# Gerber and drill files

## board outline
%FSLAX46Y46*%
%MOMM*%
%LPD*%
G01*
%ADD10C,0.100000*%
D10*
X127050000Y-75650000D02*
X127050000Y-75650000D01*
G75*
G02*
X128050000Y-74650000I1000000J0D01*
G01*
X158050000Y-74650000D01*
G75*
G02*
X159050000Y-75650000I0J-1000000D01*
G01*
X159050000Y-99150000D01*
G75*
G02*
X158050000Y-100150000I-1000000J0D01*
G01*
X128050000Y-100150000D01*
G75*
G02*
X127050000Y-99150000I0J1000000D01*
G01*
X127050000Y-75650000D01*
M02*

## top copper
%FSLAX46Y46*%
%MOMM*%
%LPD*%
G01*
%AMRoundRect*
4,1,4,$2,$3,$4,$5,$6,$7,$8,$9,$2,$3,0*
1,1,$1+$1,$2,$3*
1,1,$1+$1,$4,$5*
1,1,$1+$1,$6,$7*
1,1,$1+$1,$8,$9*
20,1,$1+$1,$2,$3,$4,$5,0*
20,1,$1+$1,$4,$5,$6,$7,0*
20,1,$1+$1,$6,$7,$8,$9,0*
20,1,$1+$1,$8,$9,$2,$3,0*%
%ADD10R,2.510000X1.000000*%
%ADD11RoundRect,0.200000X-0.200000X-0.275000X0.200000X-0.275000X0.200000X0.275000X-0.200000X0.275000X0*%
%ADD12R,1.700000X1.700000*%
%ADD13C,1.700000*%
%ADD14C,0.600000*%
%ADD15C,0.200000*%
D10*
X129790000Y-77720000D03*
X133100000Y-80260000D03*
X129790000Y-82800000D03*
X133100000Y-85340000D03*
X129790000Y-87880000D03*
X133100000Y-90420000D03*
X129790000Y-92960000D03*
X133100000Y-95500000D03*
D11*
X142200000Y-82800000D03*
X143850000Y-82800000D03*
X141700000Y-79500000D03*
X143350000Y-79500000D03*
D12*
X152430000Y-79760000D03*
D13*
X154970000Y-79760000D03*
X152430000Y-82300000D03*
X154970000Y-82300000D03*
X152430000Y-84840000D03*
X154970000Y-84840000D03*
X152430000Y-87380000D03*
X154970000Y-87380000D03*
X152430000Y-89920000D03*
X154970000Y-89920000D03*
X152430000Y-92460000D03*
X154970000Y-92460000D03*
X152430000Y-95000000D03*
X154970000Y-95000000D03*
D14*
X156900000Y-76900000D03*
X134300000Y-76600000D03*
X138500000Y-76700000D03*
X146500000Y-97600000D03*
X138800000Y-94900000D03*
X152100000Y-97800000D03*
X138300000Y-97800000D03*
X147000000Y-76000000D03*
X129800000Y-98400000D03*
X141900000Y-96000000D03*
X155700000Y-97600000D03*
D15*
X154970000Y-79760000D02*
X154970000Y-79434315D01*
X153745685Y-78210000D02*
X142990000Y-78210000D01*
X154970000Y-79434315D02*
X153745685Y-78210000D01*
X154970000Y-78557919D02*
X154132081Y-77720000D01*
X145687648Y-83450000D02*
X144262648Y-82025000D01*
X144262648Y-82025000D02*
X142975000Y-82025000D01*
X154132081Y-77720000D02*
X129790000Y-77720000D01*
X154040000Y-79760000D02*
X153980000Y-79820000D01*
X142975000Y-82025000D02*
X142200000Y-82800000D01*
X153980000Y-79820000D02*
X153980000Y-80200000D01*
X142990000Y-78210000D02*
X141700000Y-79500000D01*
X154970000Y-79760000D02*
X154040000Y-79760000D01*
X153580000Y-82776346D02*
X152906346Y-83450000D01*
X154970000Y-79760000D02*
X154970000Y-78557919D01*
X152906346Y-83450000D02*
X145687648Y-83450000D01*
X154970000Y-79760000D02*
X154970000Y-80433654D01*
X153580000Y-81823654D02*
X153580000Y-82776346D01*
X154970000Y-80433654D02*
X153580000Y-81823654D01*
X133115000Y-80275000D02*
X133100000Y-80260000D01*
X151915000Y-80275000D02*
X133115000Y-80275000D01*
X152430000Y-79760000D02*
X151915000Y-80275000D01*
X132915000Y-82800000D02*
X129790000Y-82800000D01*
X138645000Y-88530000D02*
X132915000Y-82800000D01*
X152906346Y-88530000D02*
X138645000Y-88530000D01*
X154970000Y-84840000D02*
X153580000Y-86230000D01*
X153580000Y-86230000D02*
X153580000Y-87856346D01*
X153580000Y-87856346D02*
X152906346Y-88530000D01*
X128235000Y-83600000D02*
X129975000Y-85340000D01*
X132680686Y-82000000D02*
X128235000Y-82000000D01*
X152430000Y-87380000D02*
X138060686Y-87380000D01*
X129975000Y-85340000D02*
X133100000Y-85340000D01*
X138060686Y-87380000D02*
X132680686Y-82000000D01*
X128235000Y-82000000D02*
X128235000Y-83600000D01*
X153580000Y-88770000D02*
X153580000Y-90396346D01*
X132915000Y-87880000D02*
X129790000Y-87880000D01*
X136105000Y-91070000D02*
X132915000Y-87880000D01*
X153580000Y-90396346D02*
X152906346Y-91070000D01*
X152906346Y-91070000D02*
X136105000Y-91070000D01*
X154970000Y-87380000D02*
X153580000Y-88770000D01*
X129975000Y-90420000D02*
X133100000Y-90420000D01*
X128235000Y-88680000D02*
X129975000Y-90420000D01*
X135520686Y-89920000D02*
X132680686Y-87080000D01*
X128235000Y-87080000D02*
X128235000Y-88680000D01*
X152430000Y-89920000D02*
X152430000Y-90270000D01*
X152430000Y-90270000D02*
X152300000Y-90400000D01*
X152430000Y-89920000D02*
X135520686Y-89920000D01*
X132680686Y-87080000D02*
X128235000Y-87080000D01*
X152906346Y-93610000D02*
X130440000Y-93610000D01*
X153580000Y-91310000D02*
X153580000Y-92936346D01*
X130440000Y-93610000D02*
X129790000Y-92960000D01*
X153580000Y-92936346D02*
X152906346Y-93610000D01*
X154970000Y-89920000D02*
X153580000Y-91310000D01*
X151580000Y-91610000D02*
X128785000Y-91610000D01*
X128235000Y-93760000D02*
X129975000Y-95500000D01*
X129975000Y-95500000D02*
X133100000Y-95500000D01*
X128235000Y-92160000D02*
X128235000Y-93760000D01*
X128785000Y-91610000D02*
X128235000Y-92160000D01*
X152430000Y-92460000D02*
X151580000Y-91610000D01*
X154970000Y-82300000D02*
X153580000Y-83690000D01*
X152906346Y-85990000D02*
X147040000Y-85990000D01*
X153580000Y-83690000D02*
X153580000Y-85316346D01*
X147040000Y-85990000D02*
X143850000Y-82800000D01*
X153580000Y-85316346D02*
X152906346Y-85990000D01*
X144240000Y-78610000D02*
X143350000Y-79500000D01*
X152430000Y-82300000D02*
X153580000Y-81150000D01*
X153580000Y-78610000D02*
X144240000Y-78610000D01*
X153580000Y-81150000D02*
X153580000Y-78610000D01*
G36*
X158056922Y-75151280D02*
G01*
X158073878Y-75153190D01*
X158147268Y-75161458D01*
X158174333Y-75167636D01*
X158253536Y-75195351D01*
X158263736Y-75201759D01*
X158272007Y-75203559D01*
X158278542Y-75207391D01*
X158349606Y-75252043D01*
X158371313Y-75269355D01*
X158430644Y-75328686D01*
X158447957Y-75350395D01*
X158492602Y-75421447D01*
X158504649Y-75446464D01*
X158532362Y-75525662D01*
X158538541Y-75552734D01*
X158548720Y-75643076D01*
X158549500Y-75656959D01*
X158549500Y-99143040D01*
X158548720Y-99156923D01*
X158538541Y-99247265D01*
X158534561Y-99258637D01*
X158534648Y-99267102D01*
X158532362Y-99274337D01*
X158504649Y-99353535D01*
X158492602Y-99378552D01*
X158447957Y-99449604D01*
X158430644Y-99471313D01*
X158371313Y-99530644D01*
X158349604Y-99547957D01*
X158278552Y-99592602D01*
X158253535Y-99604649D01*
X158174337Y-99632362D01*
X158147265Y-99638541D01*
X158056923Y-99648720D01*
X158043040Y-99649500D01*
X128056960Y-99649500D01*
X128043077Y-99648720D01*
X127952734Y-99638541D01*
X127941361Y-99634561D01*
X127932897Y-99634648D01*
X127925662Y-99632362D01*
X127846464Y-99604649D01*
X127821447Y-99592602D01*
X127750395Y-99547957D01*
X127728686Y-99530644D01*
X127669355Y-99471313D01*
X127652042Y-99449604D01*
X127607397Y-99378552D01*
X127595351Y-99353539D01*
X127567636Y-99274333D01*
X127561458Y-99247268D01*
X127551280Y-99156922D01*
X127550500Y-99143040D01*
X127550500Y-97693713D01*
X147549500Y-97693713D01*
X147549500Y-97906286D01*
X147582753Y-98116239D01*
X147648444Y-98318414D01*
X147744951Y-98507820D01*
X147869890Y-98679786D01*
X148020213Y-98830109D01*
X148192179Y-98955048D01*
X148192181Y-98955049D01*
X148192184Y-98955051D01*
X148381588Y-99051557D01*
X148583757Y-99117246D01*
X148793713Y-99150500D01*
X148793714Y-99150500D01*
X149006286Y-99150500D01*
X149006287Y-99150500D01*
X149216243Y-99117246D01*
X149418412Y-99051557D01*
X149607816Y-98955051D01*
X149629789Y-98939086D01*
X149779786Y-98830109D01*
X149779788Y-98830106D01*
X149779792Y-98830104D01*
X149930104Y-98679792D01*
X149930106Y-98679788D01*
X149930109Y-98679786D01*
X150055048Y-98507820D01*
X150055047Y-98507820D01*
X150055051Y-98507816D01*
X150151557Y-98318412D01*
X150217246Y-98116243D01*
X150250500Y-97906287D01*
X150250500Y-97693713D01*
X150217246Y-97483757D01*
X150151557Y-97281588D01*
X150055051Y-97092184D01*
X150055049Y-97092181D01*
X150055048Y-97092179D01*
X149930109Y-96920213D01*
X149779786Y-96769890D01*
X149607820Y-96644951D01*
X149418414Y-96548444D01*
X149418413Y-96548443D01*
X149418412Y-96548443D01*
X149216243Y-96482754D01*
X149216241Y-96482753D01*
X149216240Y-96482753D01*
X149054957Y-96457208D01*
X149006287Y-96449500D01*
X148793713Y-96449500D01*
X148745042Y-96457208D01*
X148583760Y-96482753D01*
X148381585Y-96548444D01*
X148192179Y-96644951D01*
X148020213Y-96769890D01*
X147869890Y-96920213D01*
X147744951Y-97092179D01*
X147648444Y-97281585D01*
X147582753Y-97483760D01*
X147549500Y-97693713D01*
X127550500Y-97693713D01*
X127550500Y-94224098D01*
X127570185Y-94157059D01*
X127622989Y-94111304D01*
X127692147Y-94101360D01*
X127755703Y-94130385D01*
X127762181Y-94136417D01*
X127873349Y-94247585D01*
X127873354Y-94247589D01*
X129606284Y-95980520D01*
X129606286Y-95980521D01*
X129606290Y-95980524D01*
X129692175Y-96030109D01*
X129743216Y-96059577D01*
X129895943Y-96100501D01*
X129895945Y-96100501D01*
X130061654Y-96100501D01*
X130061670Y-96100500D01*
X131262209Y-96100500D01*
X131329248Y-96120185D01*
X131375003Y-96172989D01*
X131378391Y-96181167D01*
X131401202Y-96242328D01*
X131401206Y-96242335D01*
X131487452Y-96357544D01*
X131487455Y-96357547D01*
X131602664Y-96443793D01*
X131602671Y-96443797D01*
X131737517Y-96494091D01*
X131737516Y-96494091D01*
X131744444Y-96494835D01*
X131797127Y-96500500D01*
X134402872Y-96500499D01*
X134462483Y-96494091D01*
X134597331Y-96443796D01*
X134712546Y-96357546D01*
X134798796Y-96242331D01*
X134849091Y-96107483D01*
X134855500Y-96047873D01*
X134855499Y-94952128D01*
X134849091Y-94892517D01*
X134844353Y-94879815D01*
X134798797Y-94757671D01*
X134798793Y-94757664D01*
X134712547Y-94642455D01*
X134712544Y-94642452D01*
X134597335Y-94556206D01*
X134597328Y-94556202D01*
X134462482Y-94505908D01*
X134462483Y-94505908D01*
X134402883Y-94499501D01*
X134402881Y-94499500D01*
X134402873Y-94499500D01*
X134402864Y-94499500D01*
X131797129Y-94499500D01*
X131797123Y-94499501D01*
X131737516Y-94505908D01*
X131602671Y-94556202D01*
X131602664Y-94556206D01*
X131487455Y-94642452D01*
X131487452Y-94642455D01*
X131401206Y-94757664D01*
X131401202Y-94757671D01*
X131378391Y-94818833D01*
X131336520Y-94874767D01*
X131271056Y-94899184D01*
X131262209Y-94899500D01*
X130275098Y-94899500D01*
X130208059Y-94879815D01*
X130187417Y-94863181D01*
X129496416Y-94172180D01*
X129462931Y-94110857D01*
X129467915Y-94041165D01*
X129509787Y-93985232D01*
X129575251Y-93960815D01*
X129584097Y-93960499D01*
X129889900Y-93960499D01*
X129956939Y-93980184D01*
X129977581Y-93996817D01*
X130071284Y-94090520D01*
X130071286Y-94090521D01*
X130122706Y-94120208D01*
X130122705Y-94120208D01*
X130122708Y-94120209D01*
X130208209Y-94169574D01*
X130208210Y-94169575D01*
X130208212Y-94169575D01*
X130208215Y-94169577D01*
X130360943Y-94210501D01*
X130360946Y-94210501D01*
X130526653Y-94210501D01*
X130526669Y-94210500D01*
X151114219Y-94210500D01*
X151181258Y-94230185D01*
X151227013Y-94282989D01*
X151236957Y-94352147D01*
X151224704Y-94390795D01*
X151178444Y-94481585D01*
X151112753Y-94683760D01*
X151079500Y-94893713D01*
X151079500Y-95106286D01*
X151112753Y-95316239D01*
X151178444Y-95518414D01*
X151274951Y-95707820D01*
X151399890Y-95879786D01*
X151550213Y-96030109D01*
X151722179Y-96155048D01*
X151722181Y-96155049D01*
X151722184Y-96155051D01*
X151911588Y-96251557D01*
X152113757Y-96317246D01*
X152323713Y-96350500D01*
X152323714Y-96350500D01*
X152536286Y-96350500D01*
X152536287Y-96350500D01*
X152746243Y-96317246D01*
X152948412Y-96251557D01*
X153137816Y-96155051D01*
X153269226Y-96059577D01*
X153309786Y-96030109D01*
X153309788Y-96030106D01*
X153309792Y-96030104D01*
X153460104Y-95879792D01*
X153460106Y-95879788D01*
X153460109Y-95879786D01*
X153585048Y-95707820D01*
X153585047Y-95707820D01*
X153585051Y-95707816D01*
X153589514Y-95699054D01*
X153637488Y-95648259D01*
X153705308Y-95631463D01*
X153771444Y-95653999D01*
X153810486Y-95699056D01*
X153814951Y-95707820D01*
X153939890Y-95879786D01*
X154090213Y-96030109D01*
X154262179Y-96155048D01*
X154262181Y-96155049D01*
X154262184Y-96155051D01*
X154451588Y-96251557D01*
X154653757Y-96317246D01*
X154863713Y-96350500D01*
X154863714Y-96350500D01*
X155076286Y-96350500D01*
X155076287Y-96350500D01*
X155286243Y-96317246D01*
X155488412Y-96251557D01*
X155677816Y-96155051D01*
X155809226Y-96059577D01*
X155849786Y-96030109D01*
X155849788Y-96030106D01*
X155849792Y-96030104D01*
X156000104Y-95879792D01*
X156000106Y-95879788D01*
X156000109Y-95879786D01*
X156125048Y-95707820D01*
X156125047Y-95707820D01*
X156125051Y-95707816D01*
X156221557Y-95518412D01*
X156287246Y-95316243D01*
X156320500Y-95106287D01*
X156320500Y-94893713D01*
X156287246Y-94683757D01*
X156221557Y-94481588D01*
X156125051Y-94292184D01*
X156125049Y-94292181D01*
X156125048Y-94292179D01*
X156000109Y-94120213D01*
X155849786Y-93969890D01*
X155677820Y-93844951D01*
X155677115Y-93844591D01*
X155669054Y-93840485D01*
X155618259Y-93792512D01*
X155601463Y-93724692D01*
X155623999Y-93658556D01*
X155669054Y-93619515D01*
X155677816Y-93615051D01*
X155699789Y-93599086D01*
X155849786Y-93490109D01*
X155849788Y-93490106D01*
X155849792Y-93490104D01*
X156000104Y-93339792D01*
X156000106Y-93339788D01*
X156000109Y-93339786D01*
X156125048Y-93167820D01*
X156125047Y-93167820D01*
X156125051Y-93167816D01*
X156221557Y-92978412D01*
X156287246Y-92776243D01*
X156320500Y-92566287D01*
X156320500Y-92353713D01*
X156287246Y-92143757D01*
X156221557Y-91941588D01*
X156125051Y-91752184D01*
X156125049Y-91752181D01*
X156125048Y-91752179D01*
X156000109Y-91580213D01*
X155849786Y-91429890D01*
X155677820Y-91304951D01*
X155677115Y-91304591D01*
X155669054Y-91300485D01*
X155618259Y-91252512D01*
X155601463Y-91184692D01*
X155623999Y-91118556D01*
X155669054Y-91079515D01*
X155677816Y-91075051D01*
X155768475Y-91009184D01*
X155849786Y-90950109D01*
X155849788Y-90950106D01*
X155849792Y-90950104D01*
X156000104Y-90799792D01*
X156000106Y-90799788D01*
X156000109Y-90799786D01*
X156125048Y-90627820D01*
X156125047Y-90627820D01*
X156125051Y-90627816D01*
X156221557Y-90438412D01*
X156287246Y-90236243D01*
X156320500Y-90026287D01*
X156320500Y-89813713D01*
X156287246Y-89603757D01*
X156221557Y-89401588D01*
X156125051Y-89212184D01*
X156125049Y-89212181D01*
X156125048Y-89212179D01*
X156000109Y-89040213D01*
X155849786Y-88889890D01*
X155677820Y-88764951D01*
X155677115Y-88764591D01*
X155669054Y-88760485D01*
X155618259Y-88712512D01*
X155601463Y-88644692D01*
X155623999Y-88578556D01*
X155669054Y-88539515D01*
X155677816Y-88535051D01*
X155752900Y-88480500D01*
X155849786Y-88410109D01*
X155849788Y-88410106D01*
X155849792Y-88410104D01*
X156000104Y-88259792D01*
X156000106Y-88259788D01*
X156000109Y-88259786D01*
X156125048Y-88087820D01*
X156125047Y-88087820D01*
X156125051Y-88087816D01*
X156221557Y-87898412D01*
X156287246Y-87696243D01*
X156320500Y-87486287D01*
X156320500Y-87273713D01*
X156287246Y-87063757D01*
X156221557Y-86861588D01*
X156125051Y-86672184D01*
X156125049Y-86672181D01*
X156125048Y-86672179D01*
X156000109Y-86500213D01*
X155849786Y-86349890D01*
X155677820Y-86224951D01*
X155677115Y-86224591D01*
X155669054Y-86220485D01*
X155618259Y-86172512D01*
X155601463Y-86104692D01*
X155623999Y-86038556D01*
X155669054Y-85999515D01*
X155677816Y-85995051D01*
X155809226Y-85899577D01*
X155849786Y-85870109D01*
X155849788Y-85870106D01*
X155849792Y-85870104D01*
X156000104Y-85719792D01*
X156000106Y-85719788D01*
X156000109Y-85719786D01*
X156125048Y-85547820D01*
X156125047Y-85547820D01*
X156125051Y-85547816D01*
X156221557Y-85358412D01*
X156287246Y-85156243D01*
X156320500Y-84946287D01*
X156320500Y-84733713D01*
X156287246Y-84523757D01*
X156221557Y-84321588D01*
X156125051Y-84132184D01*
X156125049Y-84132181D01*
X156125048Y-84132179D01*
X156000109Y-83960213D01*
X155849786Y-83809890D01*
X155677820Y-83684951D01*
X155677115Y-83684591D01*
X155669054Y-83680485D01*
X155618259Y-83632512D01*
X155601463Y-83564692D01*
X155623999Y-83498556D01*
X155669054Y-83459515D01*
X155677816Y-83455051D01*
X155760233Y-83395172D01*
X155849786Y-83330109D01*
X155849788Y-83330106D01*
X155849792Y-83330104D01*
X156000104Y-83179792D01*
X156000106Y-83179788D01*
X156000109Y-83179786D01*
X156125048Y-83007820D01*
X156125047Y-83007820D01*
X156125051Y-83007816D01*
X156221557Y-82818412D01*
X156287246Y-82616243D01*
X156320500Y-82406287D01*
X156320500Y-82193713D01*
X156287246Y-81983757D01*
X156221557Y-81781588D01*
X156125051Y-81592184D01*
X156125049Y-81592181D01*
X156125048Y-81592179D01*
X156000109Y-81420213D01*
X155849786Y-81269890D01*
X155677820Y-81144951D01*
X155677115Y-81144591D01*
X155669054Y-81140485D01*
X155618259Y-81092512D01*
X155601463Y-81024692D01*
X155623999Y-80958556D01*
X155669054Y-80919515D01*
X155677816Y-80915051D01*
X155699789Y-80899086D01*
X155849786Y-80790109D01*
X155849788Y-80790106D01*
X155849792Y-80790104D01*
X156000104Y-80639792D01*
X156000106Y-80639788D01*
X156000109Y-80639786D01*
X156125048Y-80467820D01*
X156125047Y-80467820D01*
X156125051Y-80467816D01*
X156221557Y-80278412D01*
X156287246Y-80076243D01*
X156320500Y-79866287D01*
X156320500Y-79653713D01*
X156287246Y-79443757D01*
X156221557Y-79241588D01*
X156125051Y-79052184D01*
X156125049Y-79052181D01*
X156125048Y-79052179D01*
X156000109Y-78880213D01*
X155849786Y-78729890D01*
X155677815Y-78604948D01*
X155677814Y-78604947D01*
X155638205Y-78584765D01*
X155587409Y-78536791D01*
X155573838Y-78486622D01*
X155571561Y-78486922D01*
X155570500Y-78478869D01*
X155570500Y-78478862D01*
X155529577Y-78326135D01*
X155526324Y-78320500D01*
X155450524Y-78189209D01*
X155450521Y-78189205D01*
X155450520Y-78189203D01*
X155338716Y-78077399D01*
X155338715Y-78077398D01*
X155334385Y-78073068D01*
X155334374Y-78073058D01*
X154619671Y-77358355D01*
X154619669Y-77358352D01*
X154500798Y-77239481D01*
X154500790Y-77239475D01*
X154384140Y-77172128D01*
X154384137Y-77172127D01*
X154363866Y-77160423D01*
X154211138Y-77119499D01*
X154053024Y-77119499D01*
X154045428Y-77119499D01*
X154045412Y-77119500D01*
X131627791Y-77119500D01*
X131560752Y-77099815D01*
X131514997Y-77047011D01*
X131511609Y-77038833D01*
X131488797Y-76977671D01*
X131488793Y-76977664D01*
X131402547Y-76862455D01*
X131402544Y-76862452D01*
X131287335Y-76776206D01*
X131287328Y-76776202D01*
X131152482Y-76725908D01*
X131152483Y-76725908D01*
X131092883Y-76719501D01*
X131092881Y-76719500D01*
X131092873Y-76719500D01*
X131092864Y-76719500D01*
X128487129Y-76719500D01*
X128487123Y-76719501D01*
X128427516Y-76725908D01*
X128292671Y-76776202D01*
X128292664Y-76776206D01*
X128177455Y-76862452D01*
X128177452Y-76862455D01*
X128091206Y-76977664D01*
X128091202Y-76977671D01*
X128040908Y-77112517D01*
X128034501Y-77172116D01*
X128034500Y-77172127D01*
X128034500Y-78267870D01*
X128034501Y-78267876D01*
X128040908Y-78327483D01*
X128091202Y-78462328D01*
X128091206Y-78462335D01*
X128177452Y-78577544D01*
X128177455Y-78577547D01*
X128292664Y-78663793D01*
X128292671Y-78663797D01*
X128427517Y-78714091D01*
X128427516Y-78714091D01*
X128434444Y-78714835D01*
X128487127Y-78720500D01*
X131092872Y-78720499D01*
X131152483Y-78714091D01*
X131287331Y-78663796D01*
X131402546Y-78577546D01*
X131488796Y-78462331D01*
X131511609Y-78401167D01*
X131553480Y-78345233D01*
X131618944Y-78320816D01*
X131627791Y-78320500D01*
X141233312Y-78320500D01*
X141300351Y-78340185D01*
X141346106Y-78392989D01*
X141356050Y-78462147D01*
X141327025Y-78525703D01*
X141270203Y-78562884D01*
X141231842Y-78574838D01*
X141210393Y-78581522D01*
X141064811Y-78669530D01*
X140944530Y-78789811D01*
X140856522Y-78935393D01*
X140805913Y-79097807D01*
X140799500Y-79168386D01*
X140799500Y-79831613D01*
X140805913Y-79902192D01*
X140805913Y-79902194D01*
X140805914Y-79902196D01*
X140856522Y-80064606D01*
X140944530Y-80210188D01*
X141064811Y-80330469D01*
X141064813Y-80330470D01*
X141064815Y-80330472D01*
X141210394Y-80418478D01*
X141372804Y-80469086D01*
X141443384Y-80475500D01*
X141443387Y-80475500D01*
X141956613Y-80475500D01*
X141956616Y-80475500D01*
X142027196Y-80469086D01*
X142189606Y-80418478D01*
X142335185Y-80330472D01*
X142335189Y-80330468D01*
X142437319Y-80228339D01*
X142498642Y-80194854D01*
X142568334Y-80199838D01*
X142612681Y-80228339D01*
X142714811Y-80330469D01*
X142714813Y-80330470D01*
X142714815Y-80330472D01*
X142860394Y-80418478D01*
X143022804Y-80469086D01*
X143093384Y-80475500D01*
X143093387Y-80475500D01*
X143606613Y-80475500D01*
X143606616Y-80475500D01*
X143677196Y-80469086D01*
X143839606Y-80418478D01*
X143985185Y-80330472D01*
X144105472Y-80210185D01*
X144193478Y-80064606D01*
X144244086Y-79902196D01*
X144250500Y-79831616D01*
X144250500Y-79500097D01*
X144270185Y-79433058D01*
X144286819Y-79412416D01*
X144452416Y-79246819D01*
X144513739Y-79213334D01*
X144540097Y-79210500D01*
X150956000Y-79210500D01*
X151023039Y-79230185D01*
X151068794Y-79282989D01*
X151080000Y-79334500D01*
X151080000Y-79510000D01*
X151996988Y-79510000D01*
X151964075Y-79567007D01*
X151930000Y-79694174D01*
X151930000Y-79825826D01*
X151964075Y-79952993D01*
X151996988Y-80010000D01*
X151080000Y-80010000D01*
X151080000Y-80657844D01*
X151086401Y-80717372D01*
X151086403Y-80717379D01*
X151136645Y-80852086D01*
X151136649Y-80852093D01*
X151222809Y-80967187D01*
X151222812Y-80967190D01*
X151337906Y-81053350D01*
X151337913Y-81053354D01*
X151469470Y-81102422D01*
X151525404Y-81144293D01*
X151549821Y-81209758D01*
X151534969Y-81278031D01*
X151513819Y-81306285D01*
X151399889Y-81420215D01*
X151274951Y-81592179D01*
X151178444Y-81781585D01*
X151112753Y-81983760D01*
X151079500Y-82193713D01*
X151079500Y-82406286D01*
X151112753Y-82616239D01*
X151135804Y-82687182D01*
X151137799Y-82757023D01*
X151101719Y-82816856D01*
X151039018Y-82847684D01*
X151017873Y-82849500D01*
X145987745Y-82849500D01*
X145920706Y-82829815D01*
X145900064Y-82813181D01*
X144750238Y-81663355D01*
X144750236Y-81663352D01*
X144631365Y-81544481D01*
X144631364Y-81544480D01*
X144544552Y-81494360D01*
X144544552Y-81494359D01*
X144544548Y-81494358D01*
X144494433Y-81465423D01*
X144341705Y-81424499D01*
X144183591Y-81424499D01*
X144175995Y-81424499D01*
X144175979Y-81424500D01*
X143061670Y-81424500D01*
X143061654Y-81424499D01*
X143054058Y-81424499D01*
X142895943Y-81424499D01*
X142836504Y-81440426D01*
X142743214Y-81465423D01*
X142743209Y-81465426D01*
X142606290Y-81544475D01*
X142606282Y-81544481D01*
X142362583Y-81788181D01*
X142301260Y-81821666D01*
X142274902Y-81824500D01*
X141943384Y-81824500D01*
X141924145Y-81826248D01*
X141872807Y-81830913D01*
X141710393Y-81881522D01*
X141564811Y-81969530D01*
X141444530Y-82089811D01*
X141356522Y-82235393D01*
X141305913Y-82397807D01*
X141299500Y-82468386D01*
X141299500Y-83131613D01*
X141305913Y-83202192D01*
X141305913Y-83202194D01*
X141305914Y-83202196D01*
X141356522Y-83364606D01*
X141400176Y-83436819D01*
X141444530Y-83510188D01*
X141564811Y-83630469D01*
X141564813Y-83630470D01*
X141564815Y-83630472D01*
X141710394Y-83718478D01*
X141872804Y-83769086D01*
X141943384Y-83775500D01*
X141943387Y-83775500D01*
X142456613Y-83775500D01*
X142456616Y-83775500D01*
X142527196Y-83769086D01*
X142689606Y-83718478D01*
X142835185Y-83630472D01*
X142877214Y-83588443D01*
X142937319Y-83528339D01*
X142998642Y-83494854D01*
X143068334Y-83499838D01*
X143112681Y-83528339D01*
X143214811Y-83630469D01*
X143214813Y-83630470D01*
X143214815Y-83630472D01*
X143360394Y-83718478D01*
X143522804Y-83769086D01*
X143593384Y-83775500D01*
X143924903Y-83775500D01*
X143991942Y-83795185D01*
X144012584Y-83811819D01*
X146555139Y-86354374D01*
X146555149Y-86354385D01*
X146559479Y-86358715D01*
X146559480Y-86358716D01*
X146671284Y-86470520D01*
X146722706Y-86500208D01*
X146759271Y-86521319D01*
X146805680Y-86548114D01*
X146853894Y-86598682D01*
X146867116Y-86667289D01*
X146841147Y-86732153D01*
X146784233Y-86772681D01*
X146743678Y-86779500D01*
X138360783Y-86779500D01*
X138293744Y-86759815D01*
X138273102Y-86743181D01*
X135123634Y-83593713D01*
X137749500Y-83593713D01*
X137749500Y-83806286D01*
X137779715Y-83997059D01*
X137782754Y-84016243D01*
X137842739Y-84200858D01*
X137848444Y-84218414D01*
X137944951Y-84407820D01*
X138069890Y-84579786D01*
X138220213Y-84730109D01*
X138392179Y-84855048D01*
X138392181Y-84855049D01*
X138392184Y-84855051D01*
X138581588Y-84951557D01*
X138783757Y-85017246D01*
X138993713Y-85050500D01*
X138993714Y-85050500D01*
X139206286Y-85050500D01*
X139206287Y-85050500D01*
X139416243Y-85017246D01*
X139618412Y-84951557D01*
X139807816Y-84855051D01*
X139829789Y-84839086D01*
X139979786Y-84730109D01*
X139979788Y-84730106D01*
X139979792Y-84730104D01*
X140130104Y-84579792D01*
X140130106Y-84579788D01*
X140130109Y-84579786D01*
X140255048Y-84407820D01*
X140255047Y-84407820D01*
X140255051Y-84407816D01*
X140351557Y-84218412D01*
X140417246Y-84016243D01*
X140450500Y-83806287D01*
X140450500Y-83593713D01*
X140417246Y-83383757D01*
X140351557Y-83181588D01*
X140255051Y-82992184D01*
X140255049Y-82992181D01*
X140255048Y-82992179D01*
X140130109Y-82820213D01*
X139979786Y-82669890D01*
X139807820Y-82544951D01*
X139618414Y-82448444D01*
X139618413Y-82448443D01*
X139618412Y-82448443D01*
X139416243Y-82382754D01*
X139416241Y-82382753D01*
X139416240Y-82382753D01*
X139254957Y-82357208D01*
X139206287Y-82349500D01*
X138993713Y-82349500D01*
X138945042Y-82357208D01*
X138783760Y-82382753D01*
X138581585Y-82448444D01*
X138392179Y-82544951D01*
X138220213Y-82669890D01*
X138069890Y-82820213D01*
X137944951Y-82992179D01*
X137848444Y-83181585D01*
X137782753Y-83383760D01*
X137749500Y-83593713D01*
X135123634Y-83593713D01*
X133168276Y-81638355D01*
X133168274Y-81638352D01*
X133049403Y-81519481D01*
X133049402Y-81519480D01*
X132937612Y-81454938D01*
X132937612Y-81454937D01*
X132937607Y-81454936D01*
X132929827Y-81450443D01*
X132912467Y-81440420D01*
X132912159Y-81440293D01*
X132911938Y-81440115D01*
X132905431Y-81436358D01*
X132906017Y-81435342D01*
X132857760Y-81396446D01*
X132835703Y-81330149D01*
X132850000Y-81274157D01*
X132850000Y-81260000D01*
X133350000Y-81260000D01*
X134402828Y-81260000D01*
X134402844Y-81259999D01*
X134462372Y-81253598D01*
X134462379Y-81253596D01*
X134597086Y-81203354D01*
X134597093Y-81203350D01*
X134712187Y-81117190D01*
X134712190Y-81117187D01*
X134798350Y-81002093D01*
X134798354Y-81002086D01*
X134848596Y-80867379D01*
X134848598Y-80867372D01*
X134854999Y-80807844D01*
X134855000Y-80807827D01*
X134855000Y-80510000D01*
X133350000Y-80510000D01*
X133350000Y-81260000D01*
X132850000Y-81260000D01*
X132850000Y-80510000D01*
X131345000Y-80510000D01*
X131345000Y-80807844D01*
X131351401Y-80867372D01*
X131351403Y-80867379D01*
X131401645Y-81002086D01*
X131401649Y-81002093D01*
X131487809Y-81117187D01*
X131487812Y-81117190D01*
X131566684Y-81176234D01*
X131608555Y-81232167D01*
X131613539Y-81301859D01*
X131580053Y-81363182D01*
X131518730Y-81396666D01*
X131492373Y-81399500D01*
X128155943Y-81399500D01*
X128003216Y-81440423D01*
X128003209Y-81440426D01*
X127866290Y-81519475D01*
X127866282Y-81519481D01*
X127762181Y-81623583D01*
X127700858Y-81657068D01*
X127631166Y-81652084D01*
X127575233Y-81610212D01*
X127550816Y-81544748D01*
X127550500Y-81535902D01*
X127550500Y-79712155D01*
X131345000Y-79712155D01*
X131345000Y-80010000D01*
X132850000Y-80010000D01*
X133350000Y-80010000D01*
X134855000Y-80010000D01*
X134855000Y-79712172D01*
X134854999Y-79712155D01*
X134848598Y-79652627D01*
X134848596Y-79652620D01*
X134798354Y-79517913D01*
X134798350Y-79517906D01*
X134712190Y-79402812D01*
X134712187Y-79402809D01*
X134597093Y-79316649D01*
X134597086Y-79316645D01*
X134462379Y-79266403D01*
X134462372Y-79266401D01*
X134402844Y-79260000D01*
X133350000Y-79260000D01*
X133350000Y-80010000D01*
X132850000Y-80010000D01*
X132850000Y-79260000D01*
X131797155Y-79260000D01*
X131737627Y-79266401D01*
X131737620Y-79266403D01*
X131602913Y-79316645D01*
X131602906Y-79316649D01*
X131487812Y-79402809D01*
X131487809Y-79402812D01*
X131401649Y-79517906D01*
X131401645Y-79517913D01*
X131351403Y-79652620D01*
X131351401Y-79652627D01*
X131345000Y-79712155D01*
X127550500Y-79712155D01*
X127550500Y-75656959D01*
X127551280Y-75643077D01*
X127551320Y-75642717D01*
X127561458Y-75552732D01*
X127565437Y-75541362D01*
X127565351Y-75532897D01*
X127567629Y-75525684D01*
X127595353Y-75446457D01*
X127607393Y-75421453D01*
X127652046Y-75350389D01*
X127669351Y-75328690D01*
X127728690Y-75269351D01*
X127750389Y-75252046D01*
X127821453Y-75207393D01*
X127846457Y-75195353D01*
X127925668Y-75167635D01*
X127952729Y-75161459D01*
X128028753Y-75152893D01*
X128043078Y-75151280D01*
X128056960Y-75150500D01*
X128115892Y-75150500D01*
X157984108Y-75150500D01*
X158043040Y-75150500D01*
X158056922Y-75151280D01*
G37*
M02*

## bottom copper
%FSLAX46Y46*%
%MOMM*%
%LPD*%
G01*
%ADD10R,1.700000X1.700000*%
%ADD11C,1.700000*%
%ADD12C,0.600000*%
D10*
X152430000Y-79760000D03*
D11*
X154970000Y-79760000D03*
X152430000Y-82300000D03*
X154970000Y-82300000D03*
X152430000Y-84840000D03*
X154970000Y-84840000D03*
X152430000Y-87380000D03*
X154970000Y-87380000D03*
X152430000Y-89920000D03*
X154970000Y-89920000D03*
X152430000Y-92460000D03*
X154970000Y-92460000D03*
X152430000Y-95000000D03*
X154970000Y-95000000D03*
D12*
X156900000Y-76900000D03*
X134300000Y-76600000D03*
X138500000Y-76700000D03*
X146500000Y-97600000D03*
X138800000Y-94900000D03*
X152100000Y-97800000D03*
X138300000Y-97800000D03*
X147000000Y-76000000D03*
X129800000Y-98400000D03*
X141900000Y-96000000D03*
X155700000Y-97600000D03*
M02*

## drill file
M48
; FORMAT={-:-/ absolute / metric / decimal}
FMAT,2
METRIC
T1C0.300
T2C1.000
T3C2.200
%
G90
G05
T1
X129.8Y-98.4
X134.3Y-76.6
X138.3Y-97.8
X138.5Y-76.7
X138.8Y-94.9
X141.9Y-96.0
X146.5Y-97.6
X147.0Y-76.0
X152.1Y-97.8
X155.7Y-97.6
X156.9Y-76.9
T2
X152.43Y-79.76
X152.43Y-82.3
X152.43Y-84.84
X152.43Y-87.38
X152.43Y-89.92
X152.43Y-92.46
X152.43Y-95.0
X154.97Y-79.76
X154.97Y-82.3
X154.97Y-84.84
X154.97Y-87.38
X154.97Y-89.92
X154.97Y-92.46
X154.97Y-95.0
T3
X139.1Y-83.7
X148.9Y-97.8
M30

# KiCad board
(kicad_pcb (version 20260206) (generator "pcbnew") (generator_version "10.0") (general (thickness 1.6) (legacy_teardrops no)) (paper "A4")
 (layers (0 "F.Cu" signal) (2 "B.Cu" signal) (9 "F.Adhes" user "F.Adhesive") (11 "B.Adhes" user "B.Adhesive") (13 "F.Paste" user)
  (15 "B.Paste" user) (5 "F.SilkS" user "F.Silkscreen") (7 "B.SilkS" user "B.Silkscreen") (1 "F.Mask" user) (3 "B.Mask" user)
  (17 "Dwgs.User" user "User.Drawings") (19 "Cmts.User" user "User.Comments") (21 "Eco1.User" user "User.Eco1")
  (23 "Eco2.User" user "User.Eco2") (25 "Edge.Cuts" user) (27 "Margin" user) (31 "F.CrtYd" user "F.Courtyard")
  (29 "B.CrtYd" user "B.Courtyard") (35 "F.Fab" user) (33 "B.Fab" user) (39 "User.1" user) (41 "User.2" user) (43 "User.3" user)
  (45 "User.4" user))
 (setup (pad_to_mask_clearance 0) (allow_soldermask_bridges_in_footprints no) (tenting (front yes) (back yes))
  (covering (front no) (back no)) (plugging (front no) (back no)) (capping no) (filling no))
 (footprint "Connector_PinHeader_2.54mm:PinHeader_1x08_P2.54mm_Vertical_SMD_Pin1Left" (layer "F.Cu") (at 131.445 86.61)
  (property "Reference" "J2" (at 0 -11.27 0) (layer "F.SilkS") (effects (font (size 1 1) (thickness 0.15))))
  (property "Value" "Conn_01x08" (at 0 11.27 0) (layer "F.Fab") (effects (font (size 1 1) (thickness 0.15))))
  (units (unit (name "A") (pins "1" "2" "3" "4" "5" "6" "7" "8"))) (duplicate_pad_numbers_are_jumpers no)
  (pad "1" smd rect (at -1.655 -8.89) (size 2.51 1) (layers "F.Cu" "F.Mask" "F.Paste") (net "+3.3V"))
  (pad "2" smd rect (at 1.655 -6.35) (size 2.51 1) (layers "F.Cu" "F.Mask" "F.Paste") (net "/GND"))
  (pad "3" smd rect (at -1.655 -3.81) (size 2.51 1) (layers "F.Cu" "F.Mask" "F.Paste") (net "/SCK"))
  (pad "4" smd rect (at 1.655 -1.27) (size 2.51 1) (layers "F.Cu" "F.Mask" "F.Paste") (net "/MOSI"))
  (pad "5" smd rect (at -1.655 1.27) (size 2.51 1) (layers "F.Cu" "F.Mask" "F.Paste") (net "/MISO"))
  (pad "6" smd rect (at 1.655 3.81) (size 2.51 1) (layers "F.Cu" "F.Mask" "F.Paste") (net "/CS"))
  (pad "7" smd rect (at -1.655 6.35) (size 2.51 1) (layers "F.Cu" "F.Mask" "F.Paste") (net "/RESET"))
  (pad "8" smd rect (at 1.655 8.89) (size 2.51 1) (layers "F.Cu" "F.Mask" "F.Paste") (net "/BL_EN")))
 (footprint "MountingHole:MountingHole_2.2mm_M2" (layer "F.Cu") (at 139.1 83.7)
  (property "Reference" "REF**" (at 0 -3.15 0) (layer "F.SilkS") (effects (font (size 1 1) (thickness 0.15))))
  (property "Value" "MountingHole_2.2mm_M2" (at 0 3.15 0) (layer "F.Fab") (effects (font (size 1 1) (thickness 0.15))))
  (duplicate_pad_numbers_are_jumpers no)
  (pad "" np_thru_hole circle (at 0 0) (size 2.2 2.2) (drill 2.2) (layers "*.Cu" "*.Mask")))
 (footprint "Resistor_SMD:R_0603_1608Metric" (layer "F.Cu") (at 143.025 82.8)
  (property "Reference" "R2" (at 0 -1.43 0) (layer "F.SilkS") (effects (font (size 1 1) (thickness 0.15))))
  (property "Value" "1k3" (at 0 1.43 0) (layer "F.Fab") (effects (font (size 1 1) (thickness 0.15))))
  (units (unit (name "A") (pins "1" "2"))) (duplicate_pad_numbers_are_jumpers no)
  (pad "1" smd roundrect (at -0.825 0) (size 0.8 0.95) (layers "F.Cu" "F.Mask" "F.Paste") (roundrect_rratio 0.25) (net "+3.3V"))
  (pad "2" smd roundrect (at 0.825 0) (size 0.8 0.95) (layers "F.Cu" "F.Mask" "F.Paste") (roundrect_rratio 0.25) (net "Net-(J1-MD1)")))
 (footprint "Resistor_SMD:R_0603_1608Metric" (layer "F.Cu") (at 142.525 79.5)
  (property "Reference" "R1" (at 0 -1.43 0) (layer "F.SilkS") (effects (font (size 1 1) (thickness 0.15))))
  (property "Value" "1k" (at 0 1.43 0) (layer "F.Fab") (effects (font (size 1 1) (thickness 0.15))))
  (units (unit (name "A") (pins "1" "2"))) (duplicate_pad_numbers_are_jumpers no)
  (pad "1" smd roundrect (at -0.825 0) (size 0.8 0.95) (layers "F.Cu" "F.Mask" "F.Paste") (roundrect_rratio 0.25) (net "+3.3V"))
  (pad "2" smd roundrect (at 0.825 0) (size 0.8 0.95) (layers "F.Cu" "F.Mask" "F.Paste") (roundrect_rratio 0.25) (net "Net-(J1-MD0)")))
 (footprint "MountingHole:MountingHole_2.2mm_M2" (layer "F.Cu") (at 148.9 97.8)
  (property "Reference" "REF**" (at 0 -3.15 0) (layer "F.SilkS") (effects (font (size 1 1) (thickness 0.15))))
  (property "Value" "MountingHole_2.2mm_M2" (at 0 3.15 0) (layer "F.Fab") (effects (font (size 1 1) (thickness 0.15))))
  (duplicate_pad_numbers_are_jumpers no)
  (pad "" np_thru_hole circle (at 0 0) (size 2.2 2.2) (drill 2.2) (layers "*.Cu" "*.Mask")))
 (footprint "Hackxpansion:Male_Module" (layer "F.Cu") (at 152.43 79.76)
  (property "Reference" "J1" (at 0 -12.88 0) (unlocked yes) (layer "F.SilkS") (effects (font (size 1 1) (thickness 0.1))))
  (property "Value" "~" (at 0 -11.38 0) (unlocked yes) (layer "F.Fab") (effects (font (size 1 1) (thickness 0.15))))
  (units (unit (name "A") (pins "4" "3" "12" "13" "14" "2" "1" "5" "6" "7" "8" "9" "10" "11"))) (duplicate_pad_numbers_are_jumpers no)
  (fp_rect (start -25.38 -5.11) (end 6.62 20.39) (radius 1) (stroke (width 0.1) (type solid)) (fill no) (layer "Edge.Cuts"))
  (pad "1" thru_hole rect (at 0 0) (size 1.7 1.7) (drill 1) (layers "*.Cu" "*.Mask") (remove_unused_layers no) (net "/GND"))
  (pad "2" thru_hole circle (at 2.54 0) (size 1.7 1.7) (drill 1) (layers "*.Cu" "*.Mask") (remove_unused_layers no) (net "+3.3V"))
  (pad "3" thru_hole circle (at 0 2.54) (size 1.7 1.7) (drill 1) (layers "*.Cu" "*.Mask") (remove_unused_layers no) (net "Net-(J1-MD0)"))
  (pad "4" thru_hole circle (at 2.54 2.54) (size 1.7 1.7) (drill 1) (layers "*.Cu" "*.Mask") (remove_unused_layers no) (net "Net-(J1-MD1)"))
  (pad "5" thru_hole circle (at 0 5.08) (size 1.7 1.7) (drill 1) (layers "*.Cu" "*.Mask") (remove_unused_layers no)
   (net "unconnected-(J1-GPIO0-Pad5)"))
  (pad "6" thru_hole circle (at 2.54 5.08) (size 1.7 1.7) (drill 1) (layers "*.Cu" "*.Mask") (remove_unused_layers no) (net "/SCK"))
  (pad "7" thru_hole circle (at 0 7.62) (size 1.7 1.7) (drill 1) (layers "*.Cu" "*.Mask") (remove_unused_layers no) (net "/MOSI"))
  (pad "8" thru_hole circle (at 2.54 7.62) (size 1.7 1.7) (drill 1) (layers "*.Cu" "*.Mask") (remove_unused_layers no) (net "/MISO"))
  (pad "9" thru_hole circle (at 0 10.16) (size 1.7 1.7) (drill 1) (layers "*.Cu" "*.Mask") (remove_unused_layers no) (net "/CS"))
  (pad "10" thru_hole circle (at 2.54 10.16) (size 1.7 1.7) (drill 1) (layers "*.Cu" "*.Mask") (remove_unused_layers no) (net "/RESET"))
  (pad "11" thru_hole circle (at 0 12.7) (size 1.7 1.7) (drill 1) (layers "*.Cu" "*.Mask") (remove_unused_layers no) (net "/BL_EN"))
  (pad "12" thru_hole circle (at 2.54 12.7) (size 1.7 1.7) (drill 1) (layers "*.Cu" "*.Mask") (remove_unused_layers no)
   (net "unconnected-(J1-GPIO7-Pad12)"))
  (pad "13" thru_hole circle (at 0 15.24) (size 1.7 1.7) (drill 1) (layers "*.Cu" "*.Mask") (remove_unused_layers no)
   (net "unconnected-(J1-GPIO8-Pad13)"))
  (pad "14" thru_hole circle (at 2.54 15.24) (size 1.7 1.7) (drill 1) (layers "*.Cu" "*.Mask") (remove_unused_layers no)
   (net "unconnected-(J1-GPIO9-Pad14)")))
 (segment (start 154.97 79.76) (end 154.97 79.434315) (width 0.2) (layer "F.Cu") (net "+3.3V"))
 (segment (start 153.745685 78.21) (end 142.99 78.21) (width 0.2) (layer "F.Cu") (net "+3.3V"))
 (segment (start 154.97 79.434315) (end 153.745685 78.21) (width 0.2) (layer "F.Cu") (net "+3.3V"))
 (segment (start 154.97 78.557919) (end 154.132081 77.72) (width 0.2) (layer "F.Cu") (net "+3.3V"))
 (segment (start 145.687648 83.45) (end 144.262648 82.025) (width 0.2) (layer "F.Cu") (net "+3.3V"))
 (segment (start 144.262648 82.025) (end 142.975 82.025) (width 0.2) (layer "F.Cu") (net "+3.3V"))
 (segment (start 154.132081 77.72) (end 129.79 77.72) (width 0.2) (layer "F.Cu") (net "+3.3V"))
 (segment (start 154.04 79.76) (end 153.98 79.82) (width 0.2) (layer "F.Cu") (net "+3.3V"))
 (segment (start 142.975 82.025) (end 142.2 82.8) (width 0.2) (layer "F.Cu") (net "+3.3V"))
 (segment (start 153.98 79.82) (end 153.98 80.2) (width 0.2) (layer "F.Cu") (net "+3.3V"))
 (segment (start 142.99 78.21) (end 141.7 79.5) (width 0.2) (layer "F.Cu") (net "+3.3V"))
 (segment (start 154.97 79.76) (end 154.04 79.76) (width 0.2) (layer "F.Cu") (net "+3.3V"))
 (segment (start 153.58 82.776346) (end 152.906346 83.45) (width 0.2) (layer "F.Cu") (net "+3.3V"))
 (segment (start 154.97 79.76) (end 154.97 78.557919) (width 0.2) (layer "F.Cu") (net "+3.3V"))
 (segment (start 152.906346 83.45) (end 145.687648 83.45) (width 0.2) (layer "F.Cu") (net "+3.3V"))
 (segment (start 154.97 79.76) (end 154.97 80.433654) (width 0.2) (layer "F.Cu") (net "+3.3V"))
 (segment (start 153.58 81.823654) (end 153.58 82.776346) (width 0.2) (layer "F.Cu") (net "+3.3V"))
 (segment (start 154.97 80.433654) (end 153.58 81.823654) (width 0.2) (layer "F.Cu") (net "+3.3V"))
 (segment (start 133.115 80.275) (end 133.1 80.26) (width 0.2) (layer "F.Cu") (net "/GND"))
 (segment (start 151.915 80.275) (end 133.115 80.275) (width 0.2) (layer "F.Cu") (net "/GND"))
 (segment (start 152.43 79.76) (end 151.915 80.275) (width 0.2) (layer "F.Cu") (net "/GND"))
 (via (at 156.9 76.9) (size 0.6) (drill 0.3) (layers "F.Cu" "B.Cu") (free yes) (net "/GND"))
 (via (at 134.3 76.6) (size 0.6) (drill 0.3) (layers "F.Cu" "B.Cu") (free yes) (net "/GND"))
 (via (at 138.5 76.7) (size 0.6) (drill 0.3) (layers "F.Cu" "B.Cu") (free yes) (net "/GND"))
 (via (at 146.5 97.6) (size 0.6) (drill 0.3) (layers "F.Cu" "B.Cu") (free yes) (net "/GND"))
 (via (at 138.8 94.9) (size 0.6) (drill 0.3) (layers "F.Cu" "B.Cu") (free yes) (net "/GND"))
 (via (at 152.1 97.8) (size 0.6) (drill 0.3) (layers "F.Cu" "B.Cu") (free yes) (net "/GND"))
 (via (at 138.3 97.8) (size 0.6) (drill 0.3) (layers "F.Cu" "B.Cu") (free yes) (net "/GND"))
 (via (at 147 76) (size 0.6) (drill 0.3) (layers "F.Cu" "B.Cu") (free yes) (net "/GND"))
 (via (at 129.8 98.4) (size 0.6) (drill 0.3) (layers "F.Cu" "B.Cu") (free yes) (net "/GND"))
 (via (at 141.9 96) (size 0.6) (drill 0.3) (layers "F.Cu" "B.Cu") (free yes) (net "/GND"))
 (via (at 155.7 97.6) (size 0.6) (drill 0.3) (layers "F.Cu" "B.Cu") (free yes) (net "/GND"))
 (segment (start 132.915 82.8) (end 129.79 82.8) (width 0.2) (layer "F.Cu") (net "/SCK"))
 (segment (start 138.645 88.53) (end 132.915 82.8) (width 0.2) (layer "F.Cu") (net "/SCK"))
 (segment (start 152.906346 88.53) (end 138.645 88.53) (width 0.2) (layer "F.Cu") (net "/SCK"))
 (segment (start 154.97 84.84) (end 153.58 86.23) (width 0.2) (layer "F.Cu") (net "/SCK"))
 (segment (start 153.58 86.23) (end 153.58 87.856346) (width 0.2) (layer "F.Cu") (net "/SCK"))
 (segment (start 153.58 87.856346) (end 152.906346 88.53) (width 0.2) (layer "F.Cu") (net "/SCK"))
 (segment (start 128.235 83.6) (end 129.975 85.34) (width 0.2) (layer "F.Cu") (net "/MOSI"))
 (segment (start 132.680686 82) (end 128.235 82) (width 0.2) (layer "F.Cu") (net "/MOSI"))
 (segment (start 152.43 87.38) (end 138.060686 87.38) (width 0.2) (layer "F.Cu") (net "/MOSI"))
 (segment (start 129.975 85.34) (end 133.1 85.34) (width 0.2) (layer "F.Cu") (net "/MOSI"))
 (segment (start 138.060686 87.38) (end 132.680686 82) (width 0.2) (layer "F.Cu") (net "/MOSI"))
 (segment (start 128.235 82) (end 128.235 83.6) (width 0.2) (layer "F.Cu") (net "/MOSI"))
 (segment (start 153.58 88.77) (end 153.58 90.396346) (width 0.2) (layer "F.Cu") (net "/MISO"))
 (segment (start 132.915 87.88) (end 129.79 87.88) (width 0.2) (layer "F.Cu") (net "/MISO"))
 (segment (start 136.105 91.07) (end 132.915 87.88) (width 0.2) (layer "F.Cu") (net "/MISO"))
 (segment (start 153.58 90.396346) (end 152.906346 91.07) (width 0.2) (layer "F.Cu") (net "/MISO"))
 (segment (start 152.906346 91.07) (end 136.105 91.07) (width 0.2) (layer "F.Cu") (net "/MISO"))
 (segment (start 154.97 87.38) (end 153.58 88.77) (width 0.2) (layer "F.Cu") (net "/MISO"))
 (segment (start 129.975 90.42) (end 133.1 90.42) (width 0.2) (layer "F.Cu") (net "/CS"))
 (segment (start 128.235 88.68) (end 129.975 90.42) (width 0.2) (layer "F.Cu") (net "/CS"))
 (segment (start 135.520686 89.92) (end 132.680686 87.08) (width 0.2) (layer "F.Cu") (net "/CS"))
 (segment (start 128.235 87.08) (end 128.235 88.68) (width 0.2) (layer "F.Cu") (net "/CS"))
 (segment (start 152.43 89.92) (end 152.43 90.27) (width 0.2) (layer "F.Cu") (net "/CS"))
 (segment (start 152.43 90.27) (end 152.3 90.4) (width 0.2) (layer "F.Cu") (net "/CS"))
 (segment (start 152.43 89.92) (end 135.520686 89.92) (width 0.2) (layer "F.Cu") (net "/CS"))
 (segment (start 132.680686 87.08) (end 128.235 87.08) (width 0.2) (layer "F.Cu") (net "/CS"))
 (segment (start 152.906346 93.61) (end 130.44 93.61) (width 0.2) (layer "F.Cu") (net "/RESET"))
 (segment (start 153.58 91.31) (end 153.58 92.936346) (width 0.2) (layer "F.Cu") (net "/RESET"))
 (segment (start 130.44 93.61) (end 129.79 92.96) (width 0.2) (layer "F.Cu") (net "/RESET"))
 (segment (start 153.58 92.936346) (end 152.906346 93.61) (width 0.2) (layer "F.Cu") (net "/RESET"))
 (segment (start 154.97 89.92) (end 153.58 91.31) (width 0.2) (layer "F.Cu") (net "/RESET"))
 (segment (start 151.58 91.61) (end 128.785 91.61) (width 0.2) (layer "F.Cu") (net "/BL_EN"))
 (segment (start 128.235 93.76) (end 129.975 95.5) (width 0.2) (layer "F.Cu") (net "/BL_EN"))
 (segment (start 129.975 95.5) (end 133.1 95.5) (width 0.2) (layer "F.Cu") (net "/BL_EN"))
 (segment (start 128.235 92.16) (end 128.235 93.76) (width 0.2) (layer "F.Cu") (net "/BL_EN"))
 (segment (start 128.785 91.61) (end 128.235 92.16) (width 0.2) (layer "F.Cu") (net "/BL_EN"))
 (segment (start 152.43 92.46) (end 151.58 91.61) (width 0.2) (layer "F.Cu") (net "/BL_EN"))
 (segment (start 154.97 82.3) (end 153.58 83.69) (width 0.2) (layer "F.Cu") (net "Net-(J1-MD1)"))
 (segment (start 152.906346 85.99) (end 147.04 85.99) (width 0.2) (layer "F.Cu") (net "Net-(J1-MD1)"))
 (segment (start 153.58 83.69) (end 153.58 85.316346) (width 0.2) (layer "F.Cu") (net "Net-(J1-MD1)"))
 (segment (start 147.04 85.99) (end 143.85 82.8) (width 0.2) (layer "F.Cu") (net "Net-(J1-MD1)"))
 (segment (start 153.58 85.316346) (end 152.906346 85.99) (width 0.2) (layer "F.Cu") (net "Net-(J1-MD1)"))
 (segment (start 144.24 78.61) (end 143.35 79.5) (width 0.2) (layer "F.Cu") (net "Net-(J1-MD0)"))
 (segment (start 152.43 82.3) (end 153.58 81.15) (width 0.2) (layer "F.Cu") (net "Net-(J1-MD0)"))
 (segment (start 153.58 78.61) (end 144.24 78.61) (width 0.2) (layer "F.Cu") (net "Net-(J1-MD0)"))
 (segment (start 153.58 81.15) (end 153.58 78.61) (width 0.2) (layer "F.Cu") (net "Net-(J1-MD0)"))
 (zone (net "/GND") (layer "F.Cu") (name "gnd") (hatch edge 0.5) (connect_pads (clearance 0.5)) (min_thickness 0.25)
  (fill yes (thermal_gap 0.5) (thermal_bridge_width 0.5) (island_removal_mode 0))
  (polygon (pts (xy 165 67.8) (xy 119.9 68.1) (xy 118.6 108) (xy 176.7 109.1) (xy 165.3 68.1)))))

